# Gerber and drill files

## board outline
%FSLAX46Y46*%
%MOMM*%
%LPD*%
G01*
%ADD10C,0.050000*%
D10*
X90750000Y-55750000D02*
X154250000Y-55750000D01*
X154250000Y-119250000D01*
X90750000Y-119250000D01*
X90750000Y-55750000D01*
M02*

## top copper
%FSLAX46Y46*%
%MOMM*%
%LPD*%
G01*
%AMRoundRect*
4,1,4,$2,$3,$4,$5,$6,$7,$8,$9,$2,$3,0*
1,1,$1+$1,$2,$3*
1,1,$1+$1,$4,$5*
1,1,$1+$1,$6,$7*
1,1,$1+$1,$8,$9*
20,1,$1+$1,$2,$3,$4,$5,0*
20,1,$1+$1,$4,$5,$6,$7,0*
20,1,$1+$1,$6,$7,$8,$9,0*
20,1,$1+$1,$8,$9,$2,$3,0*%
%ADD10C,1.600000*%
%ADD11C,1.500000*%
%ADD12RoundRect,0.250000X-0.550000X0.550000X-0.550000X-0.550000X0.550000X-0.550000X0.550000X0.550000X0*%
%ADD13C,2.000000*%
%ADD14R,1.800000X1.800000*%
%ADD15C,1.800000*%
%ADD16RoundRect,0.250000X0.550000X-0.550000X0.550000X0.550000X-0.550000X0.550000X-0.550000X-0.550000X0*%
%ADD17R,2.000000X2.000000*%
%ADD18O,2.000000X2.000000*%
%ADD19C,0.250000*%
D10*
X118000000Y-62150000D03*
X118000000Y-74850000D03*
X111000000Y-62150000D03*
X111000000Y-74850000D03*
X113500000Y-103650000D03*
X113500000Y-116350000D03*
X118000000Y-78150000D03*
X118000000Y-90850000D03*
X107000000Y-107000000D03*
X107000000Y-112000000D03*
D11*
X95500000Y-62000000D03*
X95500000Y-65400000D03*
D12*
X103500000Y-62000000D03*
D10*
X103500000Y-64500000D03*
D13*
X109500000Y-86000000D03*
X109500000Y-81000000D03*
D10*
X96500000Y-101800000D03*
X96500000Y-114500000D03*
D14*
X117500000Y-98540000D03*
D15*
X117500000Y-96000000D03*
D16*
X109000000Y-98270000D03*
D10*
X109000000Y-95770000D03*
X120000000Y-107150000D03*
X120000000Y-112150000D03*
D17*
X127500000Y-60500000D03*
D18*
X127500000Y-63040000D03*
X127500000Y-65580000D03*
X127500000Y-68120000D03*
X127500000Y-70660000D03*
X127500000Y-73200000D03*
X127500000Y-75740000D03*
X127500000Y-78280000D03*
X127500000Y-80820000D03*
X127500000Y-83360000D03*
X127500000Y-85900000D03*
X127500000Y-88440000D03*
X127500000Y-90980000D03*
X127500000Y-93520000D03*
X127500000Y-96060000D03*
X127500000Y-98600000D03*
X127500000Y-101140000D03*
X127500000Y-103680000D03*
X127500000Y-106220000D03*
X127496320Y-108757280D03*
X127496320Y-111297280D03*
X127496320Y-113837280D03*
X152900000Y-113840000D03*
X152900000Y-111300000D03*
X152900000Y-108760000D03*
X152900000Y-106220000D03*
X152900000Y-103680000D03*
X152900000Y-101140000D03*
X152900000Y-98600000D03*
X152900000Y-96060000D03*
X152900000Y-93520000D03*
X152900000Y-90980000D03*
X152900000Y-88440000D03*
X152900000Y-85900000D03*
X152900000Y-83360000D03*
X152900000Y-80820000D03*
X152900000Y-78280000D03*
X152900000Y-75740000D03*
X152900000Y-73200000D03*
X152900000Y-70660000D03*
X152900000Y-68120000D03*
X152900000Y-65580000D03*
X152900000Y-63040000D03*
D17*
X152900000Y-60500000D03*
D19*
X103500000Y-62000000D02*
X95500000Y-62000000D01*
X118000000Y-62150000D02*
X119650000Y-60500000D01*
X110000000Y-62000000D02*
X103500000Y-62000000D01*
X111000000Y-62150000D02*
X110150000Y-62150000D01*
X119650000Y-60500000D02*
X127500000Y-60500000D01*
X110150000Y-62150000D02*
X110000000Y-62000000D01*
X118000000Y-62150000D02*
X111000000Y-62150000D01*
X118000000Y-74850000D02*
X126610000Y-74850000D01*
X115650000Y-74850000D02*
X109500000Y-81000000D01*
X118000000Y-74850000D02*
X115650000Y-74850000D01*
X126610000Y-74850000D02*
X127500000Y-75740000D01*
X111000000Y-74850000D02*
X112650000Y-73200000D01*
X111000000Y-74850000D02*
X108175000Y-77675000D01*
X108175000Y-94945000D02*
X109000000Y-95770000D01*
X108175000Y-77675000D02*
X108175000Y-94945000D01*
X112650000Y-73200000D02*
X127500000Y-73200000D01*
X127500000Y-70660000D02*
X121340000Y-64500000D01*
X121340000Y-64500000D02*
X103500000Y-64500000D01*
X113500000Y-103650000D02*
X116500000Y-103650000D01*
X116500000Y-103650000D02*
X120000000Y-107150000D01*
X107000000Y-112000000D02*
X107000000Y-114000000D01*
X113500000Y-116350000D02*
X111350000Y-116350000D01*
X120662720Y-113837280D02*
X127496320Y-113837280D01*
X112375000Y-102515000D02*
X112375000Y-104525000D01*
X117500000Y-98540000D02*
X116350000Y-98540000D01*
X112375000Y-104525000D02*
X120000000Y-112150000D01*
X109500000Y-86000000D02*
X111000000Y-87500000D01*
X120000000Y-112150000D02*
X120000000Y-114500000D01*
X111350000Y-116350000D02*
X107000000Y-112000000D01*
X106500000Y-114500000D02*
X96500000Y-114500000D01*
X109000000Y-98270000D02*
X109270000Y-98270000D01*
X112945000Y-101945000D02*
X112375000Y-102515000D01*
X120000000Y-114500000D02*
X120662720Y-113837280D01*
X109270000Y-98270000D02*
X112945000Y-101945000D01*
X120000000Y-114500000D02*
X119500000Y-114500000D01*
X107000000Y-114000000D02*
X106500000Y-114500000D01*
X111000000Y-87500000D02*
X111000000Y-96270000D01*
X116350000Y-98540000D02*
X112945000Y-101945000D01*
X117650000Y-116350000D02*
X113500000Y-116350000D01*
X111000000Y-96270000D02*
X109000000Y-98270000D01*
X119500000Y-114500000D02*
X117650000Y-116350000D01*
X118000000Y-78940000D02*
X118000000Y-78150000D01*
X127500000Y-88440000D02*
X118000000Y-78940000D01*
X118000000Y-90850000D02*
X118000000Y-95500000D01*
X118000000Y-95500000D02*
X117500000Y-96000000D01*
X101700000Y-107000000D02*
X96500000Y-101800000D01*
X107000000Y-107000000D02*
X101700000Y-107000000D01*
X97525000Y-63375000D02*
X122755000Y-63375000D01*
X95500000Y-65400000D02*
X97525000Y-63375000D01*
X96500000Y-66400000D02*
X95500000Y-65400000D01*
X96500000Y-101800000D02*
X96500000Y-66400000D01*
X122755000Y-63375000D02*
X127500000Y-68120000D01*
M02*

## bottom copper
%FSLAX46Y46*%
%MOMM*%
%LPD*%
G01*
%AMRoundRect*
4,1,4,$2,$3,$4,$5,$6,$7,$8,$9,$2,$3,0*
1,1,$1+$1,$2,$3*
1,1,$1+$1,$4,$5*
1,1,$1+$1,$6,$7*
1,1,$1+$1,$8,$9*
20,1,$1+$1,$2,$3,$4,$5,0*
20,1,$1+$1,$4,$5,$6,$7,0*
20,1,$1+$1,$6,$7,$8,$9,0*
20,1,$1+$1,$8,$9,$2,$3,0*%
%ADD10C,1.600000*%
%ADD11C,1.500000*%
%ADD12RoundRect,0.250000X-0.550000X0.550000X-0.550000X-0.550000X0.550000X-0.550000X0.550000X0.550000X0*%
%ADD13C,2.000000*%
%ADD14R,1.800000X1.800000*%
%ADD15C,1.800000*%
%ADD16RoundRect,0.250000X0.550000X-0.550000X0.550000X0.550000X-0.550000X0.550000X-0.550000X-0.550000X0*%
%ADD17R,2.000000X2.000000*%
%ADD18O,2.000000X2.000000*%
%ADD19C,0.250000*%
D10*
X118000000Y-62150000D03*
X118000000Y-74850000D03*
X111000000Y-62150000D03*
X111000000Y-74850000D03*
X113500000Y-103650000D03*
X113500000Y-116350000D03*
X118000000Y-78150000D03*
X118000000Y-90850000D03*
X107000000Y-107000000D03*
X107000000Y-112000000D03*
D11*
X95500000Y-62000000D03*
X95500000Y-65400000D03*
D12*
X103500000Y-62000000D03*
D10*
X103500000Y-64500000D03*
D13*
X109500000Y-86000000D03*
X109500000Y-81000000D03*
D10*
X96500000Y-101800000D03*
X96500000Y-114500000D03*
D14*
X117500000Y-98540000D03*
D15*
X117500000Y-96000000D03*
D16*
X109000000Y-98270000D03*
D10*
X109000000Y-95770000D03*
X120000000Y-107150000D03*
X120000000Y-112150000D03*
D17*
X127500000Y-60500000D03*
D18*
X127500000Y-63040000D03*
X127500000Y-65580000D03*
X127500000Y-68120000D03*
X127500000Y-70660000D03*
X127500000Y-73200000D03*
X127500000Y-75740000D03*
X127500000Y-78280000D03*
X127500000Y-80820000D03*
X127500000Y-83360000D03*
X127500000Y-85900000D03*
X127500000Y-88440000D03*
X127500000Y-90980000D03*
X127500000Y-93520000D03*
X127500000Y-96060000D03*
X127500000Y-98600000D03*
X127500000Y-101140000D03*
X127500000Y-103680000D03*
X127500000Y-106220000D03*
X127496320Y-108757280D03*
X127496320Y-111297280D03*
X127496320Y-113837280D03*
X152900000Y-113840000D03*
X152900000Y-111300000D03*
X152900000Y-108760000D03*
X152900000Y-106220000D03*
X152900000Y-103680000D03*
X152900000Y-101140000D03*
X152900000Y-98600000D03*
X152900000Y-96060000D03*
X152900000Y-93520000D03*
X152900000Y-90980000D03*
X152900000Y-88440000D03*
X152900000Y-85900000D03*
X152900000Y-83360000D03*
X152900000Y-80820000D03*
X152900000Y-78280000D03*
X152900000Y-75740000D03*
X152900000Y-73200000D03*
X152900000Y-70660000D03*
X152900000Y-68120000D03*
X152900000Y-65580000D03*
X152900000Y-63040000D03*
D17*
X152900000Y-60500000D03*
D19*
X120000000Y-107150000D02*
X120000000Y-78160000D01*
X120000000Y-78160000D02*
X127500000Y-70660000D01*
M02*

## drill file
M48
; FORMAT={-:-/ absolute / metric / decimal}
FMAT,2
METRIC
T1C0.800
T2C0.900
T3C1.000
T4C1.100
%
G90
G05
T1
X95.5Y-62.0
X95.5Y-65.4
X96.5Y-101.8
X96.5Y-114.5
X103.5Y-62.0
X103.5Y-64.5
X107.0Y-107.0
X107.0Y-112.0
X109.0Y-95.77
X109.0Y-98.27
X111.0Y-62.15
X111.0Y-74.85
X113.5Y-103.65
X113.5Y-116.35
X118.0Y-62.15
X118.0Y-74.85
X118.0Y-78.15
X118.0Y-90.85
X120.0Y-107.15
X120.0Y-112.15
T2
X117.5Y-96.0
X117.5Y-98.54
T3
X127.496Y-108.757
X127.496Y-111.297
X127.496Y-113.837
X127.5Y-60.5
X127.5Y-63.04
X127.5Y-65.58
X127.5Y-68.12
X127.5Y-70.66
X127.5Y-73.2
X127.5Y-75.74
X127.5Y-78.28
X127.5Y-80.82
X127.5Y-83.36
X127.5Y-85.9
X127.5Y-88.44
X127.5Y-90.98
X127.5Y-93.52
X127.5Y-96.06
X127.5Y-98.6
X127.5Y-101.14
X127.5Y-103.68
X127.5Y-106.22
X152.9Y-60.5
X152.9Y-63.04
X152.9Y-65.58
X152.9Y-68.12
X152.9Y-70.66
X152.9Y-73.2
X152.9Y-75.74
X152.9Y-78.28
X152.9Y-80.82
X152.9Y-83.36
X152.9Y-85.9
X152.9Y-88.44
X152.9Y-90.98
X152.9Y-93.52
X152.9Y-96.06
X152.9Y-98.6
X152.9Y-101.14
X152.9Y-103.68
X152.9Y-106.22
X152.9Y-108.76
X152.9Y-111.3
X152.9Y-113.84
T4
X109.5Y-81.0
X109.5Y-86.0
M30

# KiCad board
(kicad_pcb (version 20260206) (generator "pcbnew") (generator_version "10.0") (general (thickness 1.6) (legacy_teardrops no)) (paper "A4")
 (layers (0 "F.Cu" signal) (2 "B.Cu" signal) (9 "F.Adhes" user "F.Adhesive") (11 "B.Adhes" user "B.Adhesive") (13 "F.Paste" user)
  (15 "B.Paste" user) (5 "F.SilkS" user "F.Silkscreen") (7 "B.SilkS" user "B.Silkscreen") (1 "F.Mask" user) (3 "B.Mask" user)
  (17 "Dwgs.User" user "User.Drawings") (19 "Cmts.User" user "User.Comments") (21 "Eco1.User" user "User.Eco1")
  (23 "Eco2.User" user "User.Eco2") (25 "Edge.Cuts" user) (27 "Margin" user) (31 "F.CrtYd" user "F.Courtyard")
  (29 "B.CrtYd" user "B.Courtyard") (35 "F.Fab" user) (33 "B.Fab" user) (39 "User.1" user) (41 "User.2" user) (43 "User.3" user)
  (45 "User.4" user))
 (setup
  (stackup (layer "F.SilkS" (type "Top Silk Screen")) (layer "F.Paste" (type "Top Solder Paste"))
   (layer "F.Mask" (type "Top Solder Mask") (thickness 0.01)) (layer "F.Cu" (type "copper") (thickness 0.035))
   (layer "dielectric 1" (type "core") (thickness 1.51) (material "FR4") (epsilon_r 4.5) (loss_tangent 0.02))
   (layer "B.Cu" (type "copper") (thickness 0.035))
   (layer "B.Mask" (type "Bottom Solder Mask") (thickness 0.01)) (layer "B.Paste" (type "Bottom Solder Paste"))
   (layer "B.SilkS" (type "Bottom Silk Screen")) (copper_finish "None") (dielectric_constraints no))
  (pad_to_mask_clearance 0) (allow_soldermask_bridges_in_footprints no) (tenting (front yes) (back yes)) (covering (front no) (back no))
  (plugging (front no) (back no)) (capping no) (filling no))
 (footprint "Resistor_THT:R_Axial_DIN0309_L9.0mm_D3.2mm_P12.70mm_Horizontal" (layer "F.Cu") (at 118 62.15 -90)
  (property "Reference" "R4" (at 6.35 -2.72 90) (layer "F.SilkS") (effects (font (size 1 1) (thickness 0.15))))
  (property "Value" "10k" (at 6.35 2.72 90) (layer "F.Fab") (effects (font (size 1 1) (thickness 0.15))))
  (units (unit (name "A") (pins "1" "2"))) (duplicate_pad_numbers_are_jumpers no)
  (pad "1" thru_hole circle (at 0 0 270) (size 1.6 1.6) (drill 0.8) (layers "*.Cu" "*.Mask") (remove_unused_layers no) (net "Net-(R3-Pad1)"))
  (pad "2" thru_hole circle (at 12.7 0 270) (size 1.6 1.6) (drill 0.8) (layers "*.Cu" "*.Mask") (remove_unused_layers no)
   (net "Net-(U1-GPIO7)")))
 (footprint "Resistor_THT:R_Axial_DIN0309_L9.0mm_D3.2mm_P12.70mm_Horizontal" (layer "F.Cu") (at 111 62.15 -90)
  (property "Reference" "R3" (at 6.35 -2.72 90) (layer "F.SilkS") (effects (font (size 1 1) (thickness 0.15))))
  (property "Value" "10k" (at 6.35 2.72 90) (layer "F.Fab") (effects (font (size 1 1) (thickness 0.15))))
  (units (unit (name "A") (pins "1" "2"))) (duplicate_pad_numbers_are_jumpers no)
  (pad "1" thru_hole circle (at 0 0 270) (size 1.6 1.6) (drill 0.8) (layers "*.Cu" "*.Mask") (remove_unused_layers no) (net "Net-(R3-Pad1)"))
  (pad "2" thru_hole circle (at 12.7 0 270) (size 1.6 1.6) (drill 0.8) (layers "*.Cu" "*.Mask") (remove_unused_layers no)
   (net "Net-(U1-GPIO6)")))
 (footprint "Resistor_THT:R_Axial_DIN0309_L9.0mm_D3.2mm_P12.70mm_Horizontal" (layer "F.Cu") (at 113.5 103.65 -90)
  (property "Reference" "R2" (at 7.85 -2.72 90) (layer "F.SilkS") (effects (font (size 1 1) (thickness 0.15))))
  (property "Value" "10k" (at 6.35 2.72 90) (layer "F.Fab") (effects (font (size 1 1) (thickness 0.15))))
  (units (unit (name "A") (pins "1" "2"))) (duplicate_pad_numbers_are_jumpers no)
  (pad "1" thru_hole circle (at 0 0 270) (size 1.6 1.6) (drill 0.8) (layers "*.Cu" "*.Mask") (remove_unused_layers no)
   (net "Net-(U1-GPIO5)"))
  (pad "2" thru_hole circle (at 12.7 0 270) (size 1.6 1.6) (drill 0.8) (layers "*.Cu" "*.Mask") (remove_unused_layers no) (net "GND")))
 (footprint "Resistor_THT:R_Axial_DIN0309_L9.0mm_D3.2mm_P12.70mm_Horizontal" (layer "F.Cu") (at 118 78.15 -90)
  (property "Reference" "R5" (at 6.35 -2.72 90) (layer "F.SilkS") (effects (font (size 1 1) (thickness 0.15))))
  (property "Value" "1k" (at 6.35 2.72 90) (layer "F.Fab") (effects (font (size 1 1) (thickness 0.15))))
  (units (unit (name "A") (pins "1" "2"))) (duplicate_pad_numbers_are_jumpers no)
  (pad "1" thru_hole circle (at 0 0 270) (size 1.6 1.6) (drill 0.8) (layers "*.Cu" "*.Mask") (remove_unused_layers no)
   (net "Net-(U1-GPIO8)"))
  (pad "2" thru_hole circle (at 12.7 0 270) (size 1.6 1.6) (drill 0.8) (layers "*.Cu" "*.Mask") (remove_unused_layers no) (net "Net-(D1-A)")))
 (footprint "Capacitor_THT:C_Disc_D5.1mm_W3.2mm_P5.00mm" (layer "F.Cu") (at 107 107 -90)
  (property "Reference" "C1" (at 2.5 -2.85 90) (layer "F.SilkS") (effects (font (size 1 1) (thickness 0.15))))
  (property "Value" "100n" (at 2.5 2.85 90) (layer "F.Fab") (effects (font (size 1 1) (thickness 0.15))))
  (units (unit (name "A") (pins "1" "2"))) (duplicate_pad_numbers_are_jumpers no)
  (pad "1" thru_hole circle (at 0 0 270) (size 1.6 1.6) (drill 0.8) (layers "*.Cu" "*.Mask") (remove_unused_layers no)
   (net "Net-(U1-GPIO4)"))
  (pad "2" thru_hole circle (at 5 0 270) (size 1.6 1.6) (drill 0.8) (layers "*.Cu" "*.Mask") (remove_unused_layers no) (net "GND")))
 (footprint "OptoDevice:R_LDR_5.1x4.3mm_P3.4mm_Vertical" (layer "F.Cu") (at 95.5 62 -90)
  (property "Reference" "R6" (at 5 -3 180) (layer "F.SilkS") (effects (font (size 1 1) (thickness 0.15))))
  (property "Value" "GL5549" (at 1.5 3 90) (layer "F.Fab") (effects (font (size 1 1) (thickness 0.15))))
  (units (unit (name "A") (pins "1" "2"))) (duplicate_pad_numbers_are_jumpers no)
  (pad "1" thru_hole circle (at 0 0 270) (size 1.5 1.5) (drill 0.8) (layers "*.Cu" "*.Mask") (remove_unused_layers no) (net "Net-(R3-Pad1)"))
  (pad "2" thru_hole circle (at 3.4 0 270) (size 1.5 1.5) (drill 0.8) (layers "*.Cu" "*.Mask") (remove_unused_layers no)
   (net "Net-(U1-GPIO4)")))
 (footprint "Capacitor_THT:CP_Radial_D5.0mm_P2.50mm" (layer "F.Cu") (at 103.5 62 -90)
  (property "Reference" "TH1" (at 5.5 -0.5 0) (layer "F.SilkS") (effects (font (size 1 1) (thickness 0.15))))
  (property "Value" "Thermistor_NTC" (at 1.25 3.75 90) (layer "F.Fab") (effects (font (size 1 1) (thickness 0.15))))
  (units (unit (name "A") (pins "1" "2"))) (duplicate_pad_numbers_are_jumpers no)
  (pad "1" thru_hole roundrect (at 0 0 270) (size 1.6 1.6) (drill 0.8) (layers "*.Cu" "*.Mask") (remove_unused_layers no)
   (roundrect_rratio 0.15625) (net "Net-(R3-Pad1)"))
  (pad "2" thru_hole circle (at 2.5 0 270) (size 1.6 1.6) (drill 0.8) (layers "*.Cu" "*.Mask") (remove_unused_layers no)
   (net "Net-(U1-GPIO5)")))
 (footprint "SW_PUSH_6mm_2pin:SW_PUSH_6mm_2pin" (layer "F.Cu") (at 109.5 83.5 90)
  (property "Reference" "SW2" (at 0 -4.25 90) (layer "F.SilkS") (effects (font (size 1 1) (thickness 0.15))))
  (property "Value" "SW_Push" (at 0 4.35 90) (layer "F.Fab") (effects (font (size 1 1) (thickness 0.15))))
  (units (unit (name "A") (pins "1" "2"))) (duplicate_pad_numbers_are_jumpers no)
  (pad "1" thru_hole circle (at -2.5 0 180) (size 2 2) (drill 1.1) (layers "*.Cu" "*.Mask") (remove_unused_layers no) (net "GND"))
  (pad "2" thru_hole circle (at 2.5 0 180) (size 2 2) (drill 1.1) (layers "*.Cu" "*.Mask") (remove_unused_layers no) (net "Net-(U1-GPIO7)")))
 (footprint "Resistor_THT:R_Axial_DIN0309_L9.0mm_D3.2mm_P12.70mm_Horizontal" (layer "F.Cu") (at 96.5 101.8 -90)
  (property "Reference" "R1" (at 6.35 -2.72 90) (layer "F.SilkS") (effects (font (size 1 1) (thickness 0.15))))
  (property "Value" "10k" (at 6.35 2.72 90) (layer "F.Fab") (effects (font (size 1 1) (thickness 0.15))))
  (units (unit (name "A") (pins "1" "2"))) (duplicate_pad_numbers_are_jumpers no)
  (pad "1" thru_hole circle (at 0 0 270) (size 1.6 1.6) (drill 0.8) (layers "*.Cu" "*.Mask") (remove_unused_layers no)
   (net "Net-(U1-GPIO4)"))
  (pad "2" thru_hole circle (at 12.7 0 270) (size 1.6 1.6) (drill 0.8) (layers "*.Cu" "*.Mask") (remove_unused_layers no) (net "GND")))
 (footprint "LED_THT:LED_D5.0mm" (layer "F.Cu") (at 117.5 98.54 90)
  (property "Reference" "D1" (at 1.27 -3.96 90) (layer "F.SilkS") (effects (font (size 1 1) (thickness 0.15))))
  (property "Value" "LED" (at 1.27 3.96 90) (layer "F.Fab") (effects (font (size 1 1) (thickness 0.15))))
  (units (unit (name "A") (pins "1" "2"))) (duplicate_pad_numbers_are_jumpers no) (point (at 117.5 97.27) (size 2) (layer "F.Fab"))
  (pad "1" thru_hole rect (at 0 0 90) (size 1.8 1.8) (drill 0.9) (layers "*.Cu" "*.Mask") (remove_unused_layers no) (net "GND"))
  (pad "2" thru_hole circle (at 2.54 0 90) (size 1.8 1.8) (drill 0.9) (layers "*.Cu" "*.Mask") (remove_unused_layers no) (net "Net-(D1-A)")))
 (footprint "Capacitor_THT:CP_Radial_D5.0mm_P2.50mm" (layer "F.Cu") (at 109 98.27 90)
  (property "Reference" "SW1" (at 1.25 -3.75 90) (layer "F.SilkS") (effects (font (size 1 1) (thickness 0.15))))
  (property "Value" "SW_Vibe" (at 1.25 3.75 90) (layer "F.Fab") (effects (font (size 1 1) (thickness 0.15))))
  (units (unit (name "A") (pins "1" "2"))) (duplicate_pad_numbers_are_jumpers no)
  (pad "1" thru_hole roundrect (at 0 0 90) (size 1.6 1.6) (drill 0.8) (layers "*.Cu" "*.Mask") (remove_unused_layers no)
   (roundrect_rratio 0.15625) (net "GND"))
  (pad "2" thru_hole circle (at 2.5 0 90) (size 1.6 1.6) (drill 0.8) (layers "*.Cu" "*.Mask") (remove_unused_layers no)
   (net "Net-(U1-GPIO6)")))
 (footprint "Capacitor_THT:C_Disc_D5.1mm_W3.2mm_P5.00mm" (layer "F.Cu") (at 120 107.15 -90)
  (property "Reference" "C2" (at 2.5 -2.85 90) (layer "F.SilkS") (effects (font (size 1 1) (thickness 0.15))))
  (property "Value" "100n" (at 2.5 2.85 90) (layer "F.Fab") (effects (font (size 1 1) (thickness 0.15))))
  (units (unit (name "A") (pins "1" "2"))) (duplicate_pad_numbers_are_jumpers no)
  (pad "1" thru_hole circle (at 0 0 270) (size 1.6 1.6) (drill 0.8) (layers "*.Cu" "*.Mask") (remove_unused_layers no)
   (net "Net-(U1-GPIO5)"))
  (pad "2" thru_hole circle (at 5 0 270) (size 1.6 1.6) (drill 0.8) (layers "*.Cu" "*.Mask") (remove_unused_layers no) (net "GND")))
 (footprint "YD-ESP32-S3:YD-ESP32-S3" (layer "F.Cu") (at 126.2 58.59)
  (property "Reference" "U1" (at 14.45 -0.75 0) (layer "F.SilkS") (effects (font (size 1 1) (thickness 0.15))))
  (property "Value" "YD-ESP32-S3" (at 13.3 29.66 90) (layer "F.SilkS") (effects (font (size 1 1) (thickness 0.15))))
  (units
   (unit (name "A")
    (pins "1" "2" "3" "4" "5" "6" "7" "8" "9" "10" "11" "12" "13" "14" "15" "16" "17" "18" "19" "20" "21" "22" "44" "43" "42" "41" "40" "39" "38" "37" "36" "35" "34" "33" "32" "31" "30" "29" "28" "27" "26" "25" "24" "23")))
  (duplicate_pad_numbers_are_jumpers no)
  (pad "1" thru_hole rect (at 1.3 1.91 270) (size 2 2) (drill 1) (layers "*.Cu" "*.Mask") (remove_unused_layers no) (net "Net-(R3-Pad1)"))
  (pad "2" thru_hole oval (at 1.3 4.45 270) (size 2 2) (drill 1) (layers "*.Cu" "*.Mask") (remove_unused_layers no)
   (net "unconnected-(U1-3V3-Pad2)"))
  (pad "3" thru_hole oval (at 1.3 6.99 270) (size 2 2) (drill 1) (layers "*.Cu" "*.Mask") (remove_unused_layers no)
   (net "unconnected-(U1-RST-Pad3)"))
  (pad "4" thru_hole oval (at 1.3 9.53 270) (size 2 2) (drill 1) (layers "*.Cu" "*.Mask") (remove_unused_layers no) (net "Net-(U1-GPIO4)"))
  (pad "5" thru_hole oval (at 1.3 12.07 270) (size 2 2) (drill 1) (layers "*.Cu" "*.Mask") (remove_unused_layers no) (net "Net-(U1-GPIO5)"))
  (pad "6" thru_hole oval (at 1.3 14.61 270) (size 2 2) (drill 1) (layers "*.Cu" "*.Mask") (remove_unused_layers no) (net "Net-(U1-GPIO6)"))
  (pad "7" thru_hole oval (at 1.3 17.15 270) (size 2 2) (drill 1) (layers "*.Cu" "*.Mask") (remove_unused_layers no) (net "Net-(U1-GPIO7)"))
  (pad "8" thru_hole oval (at 1.3 19.69 270) (size 2 2) (drill 1) (layers "*.Cu" "*.Mask") (remove_unused_layers no)
   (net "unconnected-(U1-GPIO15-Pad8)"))
  (pad "9" thru_hole oval (at 1.3 22.23 270) (size 2 2) (drill 1) (layers "*.Cu" "*.Mask") (remove_unused_layers no)
   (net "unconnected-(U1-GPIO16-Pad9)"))
  (pad "10" thru_hole oval (at 1.3 24.77 270) (size 2 2) (drill 1) (layers "*.Cu" "*.Mask") (remove_unused_layers no)
   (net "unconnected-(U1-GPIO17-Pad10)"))
  (pad "11" thru_hole oval (at 1.3 27.31 270) (size 2 2) (drill 1) (layers "*.Cu" "*.Mask") (remove_unused_layers no)
   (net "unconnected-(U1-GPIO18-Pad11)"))
  (pad "12" thru_hole oval (at 1.3 29.85 270) (size 2 2) (drill 1) (layers "*.Cu" "*.Mask") (remove_unused_layers no) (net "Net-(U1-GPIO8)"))
  (pad "13" thru_hole oval (at 1.3 32.39 270) (size 2 2) (drill 1) (layers "*.Cu" "*.Mask") (remove_unused_layers no)
   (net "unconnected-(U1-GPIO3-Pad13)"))
  (pad "14" thru_hole oval (at 1.3 34.93 270) (size 2 2) (drill 1) (layers "*.Cu" "*.Mask") (remove_unused_layers no)
   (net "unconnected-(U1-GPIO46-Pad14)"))
  (pad "15" thru_hole oval (at 1.3 37.47 270) (size 2 2) (drill 1) (layers "*.Cu" "*.Mask") (remove_unused_layers no)
   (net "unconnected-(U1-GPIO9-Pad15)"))
  (pad "16" thru_hole oval (at 1.3 40.01 270) (size 2 2) (drill 1) (layers "*.Cu" "*.Mask") (remove_unused_layers no)
   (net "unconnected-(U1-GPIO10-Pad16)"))
  (pad "17" thru_hole oval (at 1.3 42.55 270) (size 2 2) (drill 1) (layers "*.Cu" "*.Mask") (remove_unused_layers no)
   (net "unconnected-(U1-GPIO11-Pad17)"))
  (pad "18" thru_hole oval (at 1.3 45.09 270) (size 2 2) (drill 1) (layers "*.Cu" "*.Mask") (remove_unused_layers no)
   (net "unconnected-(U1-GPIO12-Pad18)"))
  (pad "19" thru_hole oval (at 1.3 47.63 270) (size 2 2) (drill 1) (layers "*.Cu" "*.Mask") (remove_unused_layers no)
   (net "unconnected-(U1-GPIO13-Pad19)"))
  (pad "20" thru_hole oval (at 1.29632 50.16728 270) (size 2 2) (drill 1) (layers "*.Cu" "*.Mask") (remove_unused_layers no)
   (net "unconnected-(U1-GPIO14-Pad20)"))
  (pad "21" thru_hole oval (at 1.29632 52.70728 270) (size 2 2) (drill 1) (layers "*.Cu" "*.Mask") (remove_unused_layers no)
   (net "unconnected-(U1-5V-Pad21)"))
  (pad "22" thru_hole oval (at 1.29632 55.24728 270) (size 2 2) (drill 1) (layers "*.Cu" "*.Mask") (remove_unused_layers no) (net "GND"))
  (pad "23" thru_hole oval (at 26.7 55.25 270) (size 2 2) (drill 1) (layers "*.Cu" "*.Mask") (remove_unused_layers no)
   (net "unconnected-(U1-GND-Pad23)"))
  (pad "24" thru_hole oval (at 26.7 52.71 270) (size 2 2) (drill 1) (layers "*.Cu" "*.Mask") (remove_unused_layers no)
   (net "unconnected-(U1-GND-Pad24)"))
  (pad "25" thru_hole oval (at 26.7 50.17 270) (size 2 2) (drill 1) (layers "*.Cu" "*.Mask") (remove_unused_layers no)
   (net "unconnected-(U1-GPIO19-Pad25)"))
  (pad "26" thru_hole oval (at 26.7 47.63 270) (size 2 2) (drill 1) (layers "*.Cu" "*.Mask") (remove_unused_layers no)
   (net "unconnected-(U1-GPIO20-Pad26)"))
  (pad "27" thru_hole oval (at 26.7 45.09 270) (size 2 2) (drill 1) (layers "*.Cu" "*.Mask") (remove_unused_layers no)
   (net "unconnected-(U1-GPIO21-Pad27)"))
  (pad "28" thru_hole oval (at 26.7 42.55 270) (size 2 2) (drill 1) (layers "*.Cu" "*.Mask") (remove_unused_layers no)
   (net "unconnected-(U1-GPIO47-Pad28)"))
  (pad "29" thru_hole oval (at 26.7 40.01 270) (size 2 2) (drill 1) (layers "*.Cu" "*.Mask") (remove_unused_layers no)
   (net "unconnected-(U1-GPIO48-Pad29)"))
  (pad "30" thru_hole oval (at 26.7 37.47 270) (size 2 2) (drill 1) (layers "*.Cu" "*.Mask") (remove_unused_layers no)
   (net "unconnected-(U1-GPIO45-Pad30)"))
  (pad "31" thru_hole oval (at 26.7 34.93 270) (size 2 2) (drill 1) (layers "*.Cu" "*.Mask") (remove_unused_layers no)
   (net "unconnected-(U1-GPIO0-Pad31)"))
  (pad "32" thru_hole oval (at 26.7 32.39 270) (size 2 2) (drill 1) (layers "*.Cu" "*.Mask") (remove_unused_layers no)
   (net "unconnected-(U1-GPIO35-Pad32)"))
  (pad "33" thru_hole oval (at 26.7 29.85 270) (size 2 2) (drill 1) (layers "*.Cu" "*.Mask") (remove_unused_layers no)
   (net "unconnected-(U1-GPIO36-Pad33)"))
  (pad "34" thru_hole oval (at 26.7 27.31 270) (size 2 2) (drill 1) (layers "*.Cu" "*.Mask") (remove_unused_layers no)
   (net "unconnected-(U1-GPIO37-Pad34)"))
  (pad "35" thru_hole oval (at 26.7 24.77 270) (size 2 2) (drill 1) (layers "*.Cu" "*.Mask") (remove_unused_layers no)
   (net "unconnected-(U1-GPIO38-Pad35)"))
  (pad "36" thru_hole oval (at 26.7 22.23 270) (size 2 2) (drill 1) (layers "*.Cu" "*.Mask") (remove_unused_layers no)
   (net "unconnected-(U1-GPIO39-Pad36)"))
  (pad "37" thru_hole oval (at 26.7 19.69 270) (size 2 2) (drill 1) (layers "*.Cu" "*.Mask") (remove_unused_layers no)
   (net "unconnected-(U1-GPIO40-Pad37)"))
  (pad "38" thru_hole oval (at 26.7 17.15 270) (size 2 2) (drill 1) (layers "*.Cu" "*.Mask") (remove_unused_layers no)
   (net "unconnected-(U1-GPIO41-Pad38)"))
  (pad "39" thru_hole oval (at 26.7 14.61 270) (size 2 2) (drill 1) (layers "*.Cu" "*.Mask") (remove_unused_layers no)
   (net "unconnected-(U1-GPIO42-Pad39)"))
  (pad "40" thru_hole oval (at 26.7 12.07 270) (size 2 2) (drill 1) (layers "*.Cu" "*.Mask") (remove_unused_layers no)
   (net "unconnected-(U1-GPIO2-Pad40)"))
  (pad "41" thru_hole oval (at 26.7 9.53 270) (size 2 2) (drill 1) (layers "*.Cu" "*.Mask") (remove_unused_layers no)
   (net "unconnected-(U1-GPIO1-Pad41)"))
  (pad "42" thru_hole oval (at 26.7 6.99 270) (size 2 2) (drill 1) (layers "*.Cu" "*.Mask") (remove_unused_layers no)
   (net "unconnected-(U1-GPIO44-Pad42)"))
  (pad "43" thru_hole oval (at 26.7 4.45 270) (size 2 2) (drill 1) (layers "*.Cu" "*.Mask") (remove_unused_layers no)
   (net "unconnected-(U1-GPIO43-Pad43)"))
  (pad "44" thru_hole rect (at 26.7 1.91 270) (size 2 2) (drill 1) (layers "*.Cu" "*.Mask") (remove_unused_layers no)
   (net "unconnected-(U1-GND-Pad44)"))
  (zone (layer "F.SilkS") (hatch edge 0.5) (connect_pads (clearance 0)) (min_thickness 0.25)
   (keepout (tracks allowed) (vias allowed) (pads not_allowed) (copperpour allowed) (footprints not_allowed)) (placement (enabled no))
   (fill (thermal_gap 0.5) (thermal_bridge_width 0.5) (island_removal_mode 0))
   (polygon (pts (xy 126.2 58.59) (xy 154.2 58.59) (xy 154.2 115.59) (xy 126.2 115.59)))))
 (gr_rect (start 90.75 55.75) (end 154.25 119.25) (stroke (width 0.05) (type default)) (fill no) (layer "Edge.Cuts"))
 (segment (start 103.5 62) (end 95.5 62) (width 0.25) (layer "F.Cu") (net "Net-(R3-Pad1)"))
 (segment (start 118 62.15) (end 119.65 60.5) (width 0.25) (layer "F.Cu") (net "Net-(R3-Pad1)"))
 (segment (start 110 62) (end 103.5 62) (width 0.25) (layer "F.Cu") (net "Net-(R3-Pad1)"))
 (segment (start 111 62.15) (end 110.15 62.15) (width 0.25) (layer "F.Cu") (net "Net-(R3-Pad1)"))
 (segment (start 119.65 60.5) (end 127.5 60.5) (width 0.25) (layer "F.Cu") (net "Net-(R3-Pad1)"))
 (segment (start 110.15 62.15) (end 110 62) (width 0.25) (layer "F.Cu") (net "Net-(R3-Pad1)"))
 (segment (start 118 62.15) (end 111 62.15) (width 0.25) (layer "F.Cu") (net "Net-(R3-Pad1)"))
 (segment (start 118 74.85) (end 126.61 74.85) (width 0.25) (layer "F.Cu") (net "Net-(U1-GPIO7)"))
 (segment (start 115.65 74.85) (end 109.5 81) (width 0.25) (layer "F.Cu") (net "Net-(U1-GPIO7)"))
 (segment (start 118 74.85) (end 115.65 74.85) (width 0.25) (layer "F.Cu") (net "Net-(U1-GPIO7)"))
 (segment (start 126.61 74.85) (end 127.5 75.74) (width 0.25) (layer "F.Cu") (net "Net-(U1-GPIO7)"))
 (segment (start 111 74.85) (end 112.65 73.2) (width 0.25) (layer "F.Cu") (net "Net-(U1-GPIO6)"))
 (segment (start 111 74.85) (end 108.175 77.675) (width 0.25) (layer "F.Cu") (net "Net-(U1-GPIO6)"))
 (segment (start 108.175 94.945) (end 109 95.77) (width 0.25) (layer "F.Cu") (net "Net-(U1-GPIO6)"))
 (segment (start 108.175 77.675) (end 108.175 94.945) (width 0.25) (layer "F.Cu") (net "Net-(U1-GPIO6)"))
 (segment (start 112.65 73.2) (end 127.5 73.2) (width 0.25) (layer "F.Cu") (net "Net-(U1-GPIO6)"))
 (segment (start 127.5 70.66) (end 121.34 64.5) (width 0.25) (layer "F.Cu") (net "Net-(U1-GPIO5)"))
 (segment (start 121.34 64.5) (end 103.5 64.5) (width 0.25) (layer "F.Cu") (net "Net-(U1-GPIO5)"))
 (segment (start 113.5 103.65) (end 116.5 103.65) (width 0.25) (layer "F.Cu") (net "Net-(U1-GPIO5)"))
 (segment (start 116.5 103.65) (end 120 107.15) (width 0.25) (layer "F.Cu") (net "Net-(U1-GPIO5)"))
 (segment (start 120 107.15) (end 120 78.16) (width 0.25) (layer "B.Cu") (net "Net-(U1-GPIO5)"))
 (segment (start 120 78.16) (end 127.5 70.66) (width 0.25) (layer "B.Cu") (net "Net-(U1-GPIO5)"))
 (segment (start 107 112) (end 107 114) (width 0.25) (layer "F.Cu") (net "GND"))
 (segment (start 113.5 116.35) (end 111.35 116.35) (width 0.25) (layer "F.Cu") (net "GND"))
 (segment (start 120.66272 113.83728) (end 127.49632 113.83728) (width 0.25) (layer "F.Cu") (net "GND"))
 (segment (start 112.375 102.515) (end 112.375 104.525) (width 0.25) (layer "F.Cu") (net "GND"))
 (segment (start 117.5 98.54) (end 116.35 98.54) (width 0.25) (layer "F.Cu") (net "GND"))
 (segment (start 112.375 104.525) (end 120 112.15) (width 0.25) (layer "F.Cu") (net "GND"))
 (segment (start 109.5 86) (end 111 87.5) (width 0.25) (layer "F.Cu") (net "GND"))
 (segment (start 120 112.15) (end 120 114.5) (width 0.25) (layer "F.Cu") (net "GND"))
 (segment (start 111.35 116.35) (end 107 112) (width 0.25) (layer "F.Cu") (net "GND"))
 (segment (start 106.5 114.5) (end 96.5 114.5) (width 0.25) (layer "F.Cu") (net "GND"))
 (segment (start 109 98.27) (end 109.27 98.27) (width 0.25) (layer "F.Cu") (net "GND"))
 (segment (start 112.945 101.945) (end 112.375 102.515) (width 0.25) (layer "F.Cu") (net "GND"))
 (segment (start 120 114.5) (end 120.66272 113.83728) (width 0.25) (layer "F.Cu") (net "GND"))
 (segment (start 109.27 98.27) (end 112.945 101.945) (width 0.25) (layer "F.Cu") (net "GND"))
 (segment (start 120 114.5) (end 119.5 114.5) (width 0.25) (layer "F.Cu") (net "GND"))
 (segment (start 107 114) (end 106.5 114.5) (width 0.25) (layer "F.Cu") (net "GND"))
 (segment (start 111 87.5) (end 111 96.27) (width 0.25) (layer "F.Cu") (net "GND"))
 (segment (start 116.35 98.54) (end 112.945 101.945) (width 0.25) (layer "F.Cu") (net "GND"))
 (segment (start 117.65 116.35) (end 113.5 116.35) (width 0.25) (layer "F.Cu") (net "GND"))
 (segment (start 111 96.27) (end 109 98.27) (width 0.25) (layer "F.Cu") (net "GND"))
 (segment (start 119.5 114.5) (end 117.65 116.35) (width 0.25) (layer "F.Cu") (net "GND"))
 (segment (start 118 78.94) (end 118 78.15) (width 0.25) (layer "F.Cu") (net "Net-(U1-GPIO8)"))
 (segment (start 127.5 88.44) (end 118 78.94) (width 0.25) (layer "F.Cu") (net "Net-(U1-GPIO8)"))
 (segment (start 118 90.85) (end 118 95.5) (width 0.25) (layer "F.Cu") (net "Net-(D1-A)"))
 (segment (start 118 95.5) (end 117.5 96) (width 0.25) (layer "F.Cu") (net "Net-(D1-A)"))
 (segment (start 101.7 107) (end 96.5 101.8) (width 0.25) (layer "F.Cu") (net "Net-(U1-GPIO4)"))
 (segment (start 107 107) (end 101.7 107) (width 0.25) (layer "F.Cu") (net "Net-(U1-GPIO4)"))
 (segment (start 97.525 63.375) (end 122.755 63.375) (width 0.25) (layer "F.Cu") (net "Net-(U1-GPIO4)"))
 (segment (start 95.5 65.4) (end 97.525 63.375) (width 0.25) (layer "F.Cu") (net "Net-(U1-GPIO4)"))
 (segment (start 96.5 66.4) (end 95.5 65.4) (width 0.25) (layer "F.Cu") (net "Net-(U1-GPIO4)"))
 (segment (start 96.5 101.8) (end 96.5 66.4) (width 0.25) (layer "F.Cu") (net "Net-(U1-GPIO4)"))
 (segment (start 122.755 63.375) (end 127.5 68.12) (width 0.25) (layer "F.Cu") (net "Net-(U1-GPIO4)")))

